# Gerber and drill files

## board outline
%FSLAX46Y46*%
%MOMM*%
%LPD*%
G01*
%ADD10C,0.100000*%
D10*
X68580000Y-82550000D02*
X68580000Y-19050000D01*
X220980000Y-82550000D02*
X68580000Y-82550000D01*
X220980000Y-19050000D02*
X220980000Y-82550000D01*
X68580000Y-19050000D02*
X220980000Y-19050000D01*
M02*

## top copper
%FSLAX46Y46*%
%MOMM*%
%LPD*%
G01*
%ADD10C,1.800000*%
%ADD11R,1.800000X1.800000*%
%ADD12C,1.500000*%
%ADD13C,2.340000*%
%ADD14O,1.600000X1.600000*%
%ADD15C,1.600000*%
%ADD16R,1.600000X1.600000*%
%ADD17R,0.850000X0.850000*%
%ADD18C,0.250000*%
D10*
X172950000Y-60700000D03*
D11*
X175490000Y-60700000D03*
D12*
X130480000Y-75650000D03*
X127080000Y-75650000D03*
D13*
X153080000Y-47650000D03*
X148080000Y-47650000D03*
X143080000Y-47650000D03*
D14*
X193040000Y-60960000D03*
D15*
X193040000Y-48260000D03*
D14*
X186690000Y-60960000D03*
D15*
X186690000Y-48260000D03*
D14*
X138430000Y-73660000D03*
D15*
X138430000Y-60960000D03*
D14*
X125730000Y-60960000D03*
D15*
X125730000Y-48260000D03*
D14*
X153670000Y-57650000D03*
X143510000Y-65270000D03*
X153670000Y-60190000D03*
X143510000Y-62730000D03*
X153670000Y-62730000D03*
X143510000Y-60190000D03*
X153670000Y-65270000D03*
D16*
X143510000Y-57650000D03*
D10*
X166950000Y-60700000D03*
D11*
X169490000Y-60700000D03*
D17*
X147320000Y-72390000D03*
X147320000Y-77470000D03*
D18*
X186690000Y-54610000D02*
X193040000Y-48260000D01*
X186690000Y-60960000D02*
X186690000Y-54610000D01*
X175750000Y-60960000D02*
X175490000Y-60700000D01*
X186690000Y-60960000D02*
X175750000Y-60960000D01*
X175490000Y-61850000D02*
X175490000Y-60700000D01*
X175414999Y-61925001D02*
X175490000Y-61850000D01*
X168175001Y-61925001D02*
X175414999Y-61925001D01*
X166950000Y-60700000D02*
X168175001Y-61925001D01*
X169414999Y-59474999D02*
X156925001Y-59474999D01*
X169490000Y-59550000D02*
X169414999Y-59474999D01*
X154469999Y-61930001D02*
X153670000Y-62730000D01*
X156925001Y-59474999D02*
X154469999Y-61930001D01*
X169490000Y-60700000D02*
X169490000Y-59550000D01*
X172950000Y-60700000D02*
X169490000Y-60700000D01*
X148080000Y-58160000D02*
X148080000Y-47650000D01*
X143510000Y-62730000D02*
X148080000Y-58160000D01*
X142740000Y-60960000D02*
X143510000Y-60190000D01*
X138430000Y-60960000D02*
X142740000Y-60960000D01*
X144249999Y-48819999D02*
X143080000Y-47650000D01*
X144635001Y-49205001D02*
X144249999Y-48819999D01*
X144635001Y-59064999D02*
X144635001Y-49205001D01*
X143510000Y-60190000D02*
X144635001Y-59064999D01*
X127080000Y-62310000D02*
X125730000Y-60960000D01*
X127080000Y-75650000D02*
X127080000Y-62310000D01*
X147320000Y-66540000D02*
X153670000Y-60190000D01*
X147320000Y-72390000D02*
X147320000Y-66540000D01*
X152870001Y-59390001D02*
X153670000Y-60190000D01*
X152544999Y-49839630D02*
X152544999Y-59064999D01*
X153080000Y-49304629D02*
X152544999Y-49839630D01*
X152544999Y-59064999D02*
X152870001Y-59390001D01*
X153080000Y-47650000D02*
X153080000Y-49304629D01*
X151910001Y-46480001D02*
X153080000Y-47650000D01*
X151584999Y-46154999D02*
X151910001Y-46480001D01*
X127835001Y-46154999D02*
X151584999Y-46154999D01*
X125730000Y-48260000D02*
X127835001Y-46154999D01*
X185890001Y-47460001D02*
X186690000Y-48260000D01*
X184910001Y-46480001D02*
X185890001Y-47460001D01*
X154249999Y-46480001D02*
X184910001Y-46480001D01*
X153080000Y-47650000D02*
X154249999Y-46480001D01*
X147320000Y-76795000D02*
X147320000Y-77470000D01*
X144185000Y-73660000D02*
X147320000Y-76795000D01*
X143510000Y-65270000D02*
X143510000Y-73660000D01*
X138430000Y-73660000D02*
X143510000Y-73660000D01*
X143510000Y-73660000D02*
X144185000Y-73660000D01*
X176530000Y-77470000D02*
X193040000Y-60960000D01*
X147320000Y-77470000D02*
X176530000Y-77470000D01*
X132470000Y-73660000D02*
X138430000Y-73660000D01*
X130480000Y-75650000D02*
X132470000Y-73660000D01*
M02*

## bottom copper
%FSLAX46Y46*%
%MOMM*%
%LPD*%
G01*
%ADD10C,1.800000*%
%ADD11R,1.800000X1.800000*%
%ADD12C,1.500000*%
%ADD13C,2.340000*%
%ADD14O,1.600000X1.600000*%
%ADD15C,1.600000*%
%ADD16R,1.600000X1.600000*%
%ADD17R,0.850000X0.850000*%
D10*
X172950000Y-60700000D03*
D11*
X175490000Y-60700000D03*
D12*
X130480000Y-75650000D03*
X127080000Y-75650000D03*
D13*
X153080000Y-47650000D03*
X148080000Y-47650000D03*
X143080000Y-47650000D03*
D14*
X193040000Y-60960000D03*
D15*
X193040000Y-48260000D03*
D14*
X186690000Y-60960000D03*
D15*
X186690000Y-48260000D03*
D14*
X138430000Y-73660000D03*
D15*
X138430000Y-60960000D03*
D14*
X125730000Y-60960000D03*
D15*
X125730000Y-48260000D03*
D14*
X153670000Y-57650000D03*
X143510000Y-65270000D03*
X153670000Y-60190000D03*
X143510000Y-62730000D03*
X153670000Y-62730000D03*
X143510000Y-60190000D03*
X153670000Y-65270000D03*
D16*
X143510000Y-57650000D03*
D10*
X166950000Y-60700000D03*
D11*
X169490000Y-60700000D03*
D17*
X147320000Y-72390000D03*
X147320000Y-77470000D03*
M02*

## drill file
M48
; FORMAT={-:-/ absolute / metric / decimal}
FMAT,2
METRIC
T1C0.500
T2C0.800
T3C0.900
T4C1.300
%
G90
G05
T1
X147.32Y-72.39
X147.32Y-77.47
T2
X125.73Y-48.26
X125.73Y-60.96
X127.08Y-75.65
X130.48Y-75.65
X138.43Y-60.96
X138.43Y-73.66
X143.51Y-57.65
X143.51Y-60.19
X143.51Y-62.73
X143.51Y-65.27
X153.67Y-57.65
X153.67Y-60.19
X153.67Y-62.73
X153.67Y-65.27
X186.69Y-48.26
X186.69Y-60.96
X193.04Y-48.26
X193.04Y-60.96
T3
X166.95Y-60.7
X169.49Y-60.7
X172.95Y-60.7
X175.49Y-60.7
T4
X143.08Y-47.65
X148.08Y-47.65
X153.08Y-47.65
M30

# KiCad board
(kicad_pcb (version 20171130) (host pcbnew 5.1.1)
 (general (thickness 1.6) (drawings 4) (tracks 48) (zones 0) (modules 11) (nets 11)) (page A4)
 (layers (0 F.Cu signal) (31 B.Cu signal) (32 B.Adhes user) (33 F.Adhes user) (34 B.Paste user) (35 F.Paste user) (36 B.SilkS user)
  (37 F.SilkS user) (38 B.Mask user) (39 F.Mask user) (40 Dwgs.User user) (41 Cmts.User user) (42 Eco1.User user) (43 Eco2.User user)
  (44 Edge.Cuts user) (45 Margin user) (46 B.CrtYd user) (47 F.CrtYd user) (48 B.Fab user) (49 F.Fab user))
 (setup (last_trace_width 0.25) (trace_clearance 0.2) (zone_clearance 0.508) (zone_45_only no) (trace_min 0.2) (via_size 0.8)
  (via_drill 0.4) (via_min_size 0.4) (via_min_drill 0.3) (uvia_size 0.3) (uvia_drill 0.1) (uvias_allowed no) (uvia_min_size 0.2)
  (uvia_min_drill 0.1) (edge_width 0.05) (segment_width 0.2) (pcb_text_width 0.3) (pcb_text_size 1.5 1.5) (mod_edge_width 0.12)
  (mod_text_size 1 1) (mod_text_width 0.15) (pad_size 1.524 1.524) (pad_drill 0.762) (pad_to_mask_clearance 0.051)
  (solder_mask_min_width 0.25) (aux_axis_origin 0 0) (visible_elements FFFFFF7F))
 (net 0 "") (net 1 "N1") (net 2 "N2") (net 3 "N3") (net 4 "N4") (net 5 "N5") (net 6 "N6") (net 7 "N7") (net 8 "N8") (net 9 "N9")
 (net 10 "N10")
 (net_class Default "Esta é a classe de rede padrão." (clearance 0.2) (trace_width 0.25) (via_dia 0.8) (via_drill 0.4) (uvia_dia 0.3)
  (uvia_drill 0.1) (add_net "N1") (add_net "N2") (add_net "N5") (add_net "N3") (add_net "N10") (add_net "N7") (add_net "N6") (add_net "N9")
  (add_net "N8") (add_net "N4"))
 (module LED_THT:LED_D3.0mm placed (layer F.Cu) (at 175.49 60.7 180)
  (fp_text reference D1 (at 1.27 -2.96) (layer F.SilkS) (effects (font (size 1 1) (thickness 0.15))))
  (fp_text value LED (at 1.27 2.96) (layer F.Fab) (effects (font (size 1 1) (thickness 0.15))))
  (pad 2 thru_hole circle (at 2.54 0 180) (size 1.8 1.8) (drill 0.9) (layers *.Cu *.Mask) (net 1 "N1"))
  (pad 1 thru_hole rect (at 0 0 180) (size 1.8 1.8) (drill 0.9) (layers *.Cu *.Mask) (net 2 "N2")))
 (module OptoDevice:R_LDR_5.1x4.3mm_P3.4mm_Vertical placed (layer F.Cu) (at 127.08 75.65)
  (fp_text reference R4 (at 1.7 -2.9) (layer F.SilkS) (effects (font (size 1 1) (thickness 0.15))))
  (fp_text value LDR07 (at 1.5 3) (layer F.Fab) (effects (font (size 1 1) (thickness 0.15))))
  (pad 2 thru_hole circle (at 3.4 0) (size 1.5 1.5) (drill 0.8) (layers *.Cu *.Mask) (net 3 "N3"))
  (pad 1 thru_hole circle (at 0 0) (size 1.5 1.5) (drill 0.8) (layers *.Cu *.Mask) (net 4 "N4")))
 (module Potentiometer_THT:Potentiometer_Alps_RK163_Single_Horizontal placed (layer F.Cu) (at 153.08 47.65 90)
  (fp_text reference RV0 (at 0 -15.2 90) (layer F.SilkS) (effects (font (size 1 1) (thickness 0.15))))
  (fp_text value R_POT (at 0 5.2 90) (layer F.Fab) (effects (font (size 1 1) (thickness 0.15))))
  (pad 1 thru_hole circle (at 0 0 90) (size 2.34 2.34) (drill 1.3) (layers *.Cu *.Mask) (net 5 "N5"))
  (pad 2 thru_hole circle (at 0 -5 90) (size 2.34 2.34) (drill 1.3) (layers *.Cu *.Mask) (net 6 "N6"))
  (pad 3 thru_hole circle (at 0 -10 90) (size 2.34 2.34) (drill 1.3) (layers *.Cu *.Mask) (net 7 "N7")))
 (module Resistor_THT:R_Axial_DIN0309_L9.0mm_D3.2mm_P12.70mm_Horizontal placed (layer F.Cu) (at 193.04 48.26 270)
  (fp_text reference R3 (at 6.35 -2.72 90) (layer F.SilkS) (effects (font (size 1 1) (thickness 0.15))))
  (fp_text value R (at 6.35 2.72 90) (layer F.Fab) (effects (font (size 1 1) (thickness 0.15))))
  (pad 2 thru_hole oval (at 12.7 0 270) (size 1.6 1.6) (drill 0.8) (layers *.Cu *.Mask) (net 3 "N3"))
  (pad 1 thru_hole circle (at 0 0 270) (size 1.6 1.6) (drill 0.8) (layers *.Cu *.Mask) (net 2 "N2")))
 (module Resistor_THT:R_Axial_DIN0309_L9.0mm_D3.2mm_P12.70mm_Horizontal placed (layer F.Cu) (at 186.69 48.26 270)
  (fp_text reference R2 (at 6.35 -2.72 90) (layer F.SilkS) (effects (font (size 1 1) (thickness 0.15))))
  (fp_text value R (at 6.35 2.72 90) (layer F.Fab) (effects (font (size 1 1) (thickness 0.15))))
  (pad 2 thru_hole oval (at 12.7 0 270) (size 1.6 1.6) (drill 0.8) (layers *.Cu *.Mask) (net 2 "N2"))
  (pad 1 thru_hole circle (at 0 0 270) (size 1.6 1.6) (drill 0.8) (layers *.Cu *.Mask) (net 5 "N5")))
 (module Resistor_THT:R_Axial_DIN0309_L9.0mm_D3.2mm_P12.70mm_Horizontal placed (layer F.Cu) (at 138.43 60.96 270)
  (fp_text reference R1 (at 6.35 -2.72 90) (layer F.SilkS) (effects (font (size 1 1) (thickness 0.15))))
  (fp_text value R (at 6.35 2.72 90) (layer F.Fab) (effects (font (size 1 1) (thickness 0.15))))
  (pad 2 thru_hole oval (at 12.7 0 270) (size 1.6 1.6) (drill 0.8) (layers *.Cu *.Mask) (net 3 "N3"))
  (pad 1 thru_hole circle (at 0 0 270) (size 1.6 1.6) (drill 0.8) (layers *.Cu *.Mask) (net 7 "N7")))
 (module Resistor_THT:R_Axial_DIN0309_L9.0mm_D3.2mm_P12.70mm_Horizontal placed (layer F.Cu) (at 125.73 48.26 270)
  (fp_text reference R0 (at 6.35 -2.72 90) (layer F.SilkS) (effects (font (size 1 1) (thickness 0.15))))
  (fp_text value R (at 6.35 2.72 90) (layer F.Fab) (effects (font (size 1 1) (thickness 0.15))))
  (pad 2 thru_hole oval (at 12.7 0 270) (size 1.6 1.6) (drill 0.8) (layers *.Cu *.Mask) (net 4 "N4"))
  (pad 1 thru_hole circle (at 0 0 270) (size 1.6 1.6) (drill 0.8) (layers *.Cu *.Mask) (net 5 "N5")))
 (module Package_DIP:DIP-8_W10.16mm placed (layer F.Cu) (at 143.51 57.65)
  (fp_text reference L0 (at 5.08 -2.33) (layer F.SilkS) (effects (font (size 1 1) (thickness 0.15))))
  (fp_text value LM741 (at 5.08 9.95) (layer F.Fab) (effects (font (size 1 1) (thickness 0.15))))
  (pad 8 thru_hole oval (at 10.16 0) (size 1.6 1.6) (drill 0.8) (layers *.Cu *.Mask) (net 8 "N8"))
  (pad 4 thru_hole oval (at 0 7.62) (size 1.6 1.6) (drill 0.8) (layers *.Cu *.Mask) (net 3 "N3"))
  (pad 7 thru_hole oval (at 10.16 2.54) (size 1.6 1.6) (drill 0.8) (layers *.Cu *.Mask) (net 5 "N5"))
  (pad 3 thru_hole oval (at 0 5.08) (size 1.6 1.6) (drill 0.8) (layers *.Cu *.Mask) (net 6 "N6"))
  (pad 6 thru_hole oval (at 10.16 5.08) (size 1.6 1.6) (drill 0.8) (layers *.Cu *.Mask) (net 1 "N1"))
  (pad 2 thru_hole oval (at 0 2.54) (size 1.6 1.6) (drill 0.8) (layers *.Cu *.Mask) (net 7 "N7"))
  (pad 5 thru_hole oval (at 10.16 7.62) (size 1.6 1.6) (drill 0.8) (layers *.Cu *.Mask) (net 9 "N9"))
  (pad 1 thru_hole rect (at 0 0) (size 1.6 1.6) (drill 0.8) (layers *.Cu *.Mask) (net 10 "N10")))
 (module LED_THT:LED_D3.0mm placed (layer F.Cu) (at 169.49 60.7 180)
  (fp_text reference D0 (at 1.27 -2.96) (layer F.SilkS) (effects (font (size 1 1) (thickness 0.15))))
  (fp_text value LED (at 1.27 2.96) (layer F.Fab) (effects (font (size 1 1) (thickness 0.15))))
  (pad 2 thru_hole circle (at 2.54 0 180) (size 1.8 1.8) (drill 0.9) (layers *.Cu *.Mask) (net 2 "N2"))
  (pad 1 thru_hole rect (at 0 0 180) (size 1.8 1.8) (drill 0.9) (layers *.Cu *.Mask) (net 1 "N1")))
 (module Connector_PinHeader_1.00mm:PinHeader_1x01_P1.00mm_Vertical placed (layer F.Cu) (at 147.32 72.39)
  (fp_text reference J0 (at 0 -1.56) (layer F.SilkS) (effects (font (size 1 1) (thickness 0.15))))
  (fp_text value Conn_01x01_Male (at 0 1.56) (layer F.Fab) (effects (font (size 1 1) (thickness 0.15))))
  (pad 1 thru_hole rect (at 0 0) (size 0.85 0.85) (drill 0.5) (layers *.Cu *.Mask) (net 5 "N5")))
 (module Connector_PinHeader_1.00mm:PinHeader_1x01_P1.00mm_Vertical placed (layer F.Cu) (at 147.32 77.47)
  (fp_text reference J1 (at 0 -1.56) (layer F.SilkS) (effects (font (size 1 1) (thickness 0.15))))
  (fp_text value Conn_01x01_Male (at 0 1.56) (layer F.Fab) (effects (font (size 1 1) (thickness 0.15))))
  (pad 1 thru_hole rect (at 0 0) (size 0.85 0.85) (drill 0.5) (layers *.Cu *.Mask) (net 3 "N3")))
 (gr_line (start 68.58 82.55) (end 68.58 19.05) (layer Edge.Cuts) (width 0.1))
 (gr_line (start 220.98 82.55) (end 68.58 82.55) (layer Edge.Cuts) (width 0.1))
 (gr_line (start 220.98 19.05) (end 220.98 82.55) (layer Edge.Cuts) (width 0.1))
 (gr_line (start 68.58 19.05) (end 220.98 19.05) (layer Edge.Cuts) (width 0.1))
 (segment (start 186.69 54.61) (end 193.04 48.26) (width 0.25) (layer F.Cu) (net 2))
 (segment (start 186.69 60.96) (end 186.69 54.61) (width 0.25) (layer F.Cu) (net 2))
 (segment (start 175.75 60.96) (end 175.49 60.7) (width 0.25) (layer F.Cu) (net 2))
 (segment (start 186.69 60.96) (end 175.75 60.96) (width 0.25) (layer F.Cu) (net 2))
 (segment (start 175.49 61.85) (end 175.49 60.7) (width 0.25) (layer F.Cu) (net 2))
 (segment (start 175.414999 61.925001) (end 175.49 61.85) (width 0.25) (layer F.Cu) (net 2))
 (segment (start 168.175001 61.925001) (end 175.414999 61.925001) (width 0.25) (layer F.Cu) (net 2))
 (segment (start 166.95 60.7) (end 168.175001 61.925001) (width 0.25) (layer F.Cu) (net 2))
 (segment (start 169.414999 59.474999) (end 156.925001 59.474999) (width 0.25) (layer F.Cu) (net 1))
 (segment (start 169.49 59.55) (end 169.414999 59.474999) (width 0.25) (layer F.Cu) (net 1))
 (segment (start 154.469999 61.930001) (end 153.67 62.73) (width 0.25) (layer F.Cu) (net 1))
 (segment (start 156.925001 59.474999) (end 154.469999 61.930001) (width 0.25) (layer F.Cu) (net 1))
 (segment (start 169.49 60.7) (end 169.49 59.55) (width 0.25) (layer F.Cu) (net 1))
 (segment (start 172.95 60.7) (end 169.49 60.7) (width 0.25) (layer F.Cu) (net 1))
 (segment (start 148.08 58.16) (end 148.08 47.65) (width 0.25) (layer F.Cu) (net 6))
 (segment (start 143.51 62.73) (end 148.08 58.16) (width 0.25) (layer F.Cu) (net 6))
 (segment (start 142.74 60.96) (end 143.51 60.19) (width 0.25) (layer F.Cu) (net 7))
 (segment (start 138.43 60.96) (end 142.74 60.96) (width 0.25) (layer F.Cu) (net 7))
 (segment (start 144.249999 48.819999) (end 143.08 47.65) (width 0.25) (layer F.Cu) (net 7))
 (segment (start 144.635001 49.205001) (end 144.249999 48.819999) (width 0.25) (layer F.Cu) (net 7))
 (segment (start 144.635001 59.064999) (end 144.635001 49.205001) (width 0.25) (layer F.Cu) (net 7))
 (segment (start 143.51 60.19) (end 144.635001 59.064999) (width 0.25) (layer F.Cu) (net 7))
 (segment (start 127.08 62.31) (end 125.73 60.96) (width 0.25) (layer F.Cu) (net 4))
 (segment (start 127.08 75.65) (end 127.08 62.31) (width 0.25) (layer F.Cu) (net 4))
 (segment (start 147.32 66.54) (end 153.67 60.19) (width 0.25) (layer F.Cu) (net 5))
 (segment (start 147.32 72.39) (end 147.32 66.54) (width 0.25) (layer F.Cu) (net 5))
 (segment (start 152.870001 59.390001) (end 153.67 60.19) (width 0.25) (layer F.Cu) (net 5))
 (segment (start 152.544999 49.83963) (end 152.544999 59.064999) (width 0.25) (layer F.Cu) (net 5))
 (segment (start 153.08 49.304629) (end 152.544999 49.83963) (width 0.25) (layer F.Cu) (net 5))
 (segment (start 152.544999 59.064999) (end 152.870001 59.390001) (width 0.25) (layer F.Cu) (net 5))
 (segment (start 153.08 47.65) (end 153.08 49.304629) (width 0.25) (layer F.Cu) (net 5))
 (segment (start 151.910001 46.480001) (end 153.08 47.65) (width 0.25) (layer F.Cu) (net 5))
 (segment (start 151.584999 46.154999) (end 151.910001 46.480001) (width 0.25) (layer F.Cu) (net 5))
 (segment (start 127.835001 46.154999) (end 151.584999 46.154999) (width 0.25) (layer F.Cu) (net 5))
 (segment (start 125.73 48.26) (end 127.835001 46.154999) (width 0.25) (layer F.Cu) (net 5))
 (segment (start 185.890001 47.460001) (end 186.69 48.26) (width 0.25) (layer F.Cu) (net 5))
 (segment (start 184.910001 46.480001) (end 185.890001 47.460001) (width 0.25) (layer F.Cu) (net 5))
 (segment (start 154.249999 46.480001) (end 184.910001 46.480001) (width 0.25) (layer F.Cu) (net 5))
 (segment (start 153.08 47.65) (end 154.249999 46.480001) (width 0.25) (layer F.Cu) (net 5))
 (segment (start 147.32 76.795) (end 147.32 77.47) (width 0.25) (layer F.Cu) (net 3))
 (segment (start 144.185 73.66) (end 147.32 76.795) (width 0.25) (layer F.Cu) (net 3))
 (segment (start 143.51 65.27) (end 143.51 73.66) (width 0.25) (layer F.Cu) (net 3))
 (segment (start 138.43 73.66) (end 143.51 73.66) (width 0.25) (layer F.Cu) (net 3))
 (segment (start 143.51 73.66) (end 144.185 73.66) (width 0.25) (layer F.Cu) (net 3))
 (segment (start 176.53 77.47) (end 193.04 60.96) (width 0.25) (layer F.Cu) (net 3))
 (segment (start 147.32 77.47) (end 176.53 77.47) (width 0.25) (layer F.Cu) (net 3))
 (segment (start 132.47 73.66) (end 138.43 73.66) (width 0.25) (layer F.Cu) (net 3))
 (segment (start 130.48 75.65) (end 132.47 73.66) (width 0.25) (layer F.Cu) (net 3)))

